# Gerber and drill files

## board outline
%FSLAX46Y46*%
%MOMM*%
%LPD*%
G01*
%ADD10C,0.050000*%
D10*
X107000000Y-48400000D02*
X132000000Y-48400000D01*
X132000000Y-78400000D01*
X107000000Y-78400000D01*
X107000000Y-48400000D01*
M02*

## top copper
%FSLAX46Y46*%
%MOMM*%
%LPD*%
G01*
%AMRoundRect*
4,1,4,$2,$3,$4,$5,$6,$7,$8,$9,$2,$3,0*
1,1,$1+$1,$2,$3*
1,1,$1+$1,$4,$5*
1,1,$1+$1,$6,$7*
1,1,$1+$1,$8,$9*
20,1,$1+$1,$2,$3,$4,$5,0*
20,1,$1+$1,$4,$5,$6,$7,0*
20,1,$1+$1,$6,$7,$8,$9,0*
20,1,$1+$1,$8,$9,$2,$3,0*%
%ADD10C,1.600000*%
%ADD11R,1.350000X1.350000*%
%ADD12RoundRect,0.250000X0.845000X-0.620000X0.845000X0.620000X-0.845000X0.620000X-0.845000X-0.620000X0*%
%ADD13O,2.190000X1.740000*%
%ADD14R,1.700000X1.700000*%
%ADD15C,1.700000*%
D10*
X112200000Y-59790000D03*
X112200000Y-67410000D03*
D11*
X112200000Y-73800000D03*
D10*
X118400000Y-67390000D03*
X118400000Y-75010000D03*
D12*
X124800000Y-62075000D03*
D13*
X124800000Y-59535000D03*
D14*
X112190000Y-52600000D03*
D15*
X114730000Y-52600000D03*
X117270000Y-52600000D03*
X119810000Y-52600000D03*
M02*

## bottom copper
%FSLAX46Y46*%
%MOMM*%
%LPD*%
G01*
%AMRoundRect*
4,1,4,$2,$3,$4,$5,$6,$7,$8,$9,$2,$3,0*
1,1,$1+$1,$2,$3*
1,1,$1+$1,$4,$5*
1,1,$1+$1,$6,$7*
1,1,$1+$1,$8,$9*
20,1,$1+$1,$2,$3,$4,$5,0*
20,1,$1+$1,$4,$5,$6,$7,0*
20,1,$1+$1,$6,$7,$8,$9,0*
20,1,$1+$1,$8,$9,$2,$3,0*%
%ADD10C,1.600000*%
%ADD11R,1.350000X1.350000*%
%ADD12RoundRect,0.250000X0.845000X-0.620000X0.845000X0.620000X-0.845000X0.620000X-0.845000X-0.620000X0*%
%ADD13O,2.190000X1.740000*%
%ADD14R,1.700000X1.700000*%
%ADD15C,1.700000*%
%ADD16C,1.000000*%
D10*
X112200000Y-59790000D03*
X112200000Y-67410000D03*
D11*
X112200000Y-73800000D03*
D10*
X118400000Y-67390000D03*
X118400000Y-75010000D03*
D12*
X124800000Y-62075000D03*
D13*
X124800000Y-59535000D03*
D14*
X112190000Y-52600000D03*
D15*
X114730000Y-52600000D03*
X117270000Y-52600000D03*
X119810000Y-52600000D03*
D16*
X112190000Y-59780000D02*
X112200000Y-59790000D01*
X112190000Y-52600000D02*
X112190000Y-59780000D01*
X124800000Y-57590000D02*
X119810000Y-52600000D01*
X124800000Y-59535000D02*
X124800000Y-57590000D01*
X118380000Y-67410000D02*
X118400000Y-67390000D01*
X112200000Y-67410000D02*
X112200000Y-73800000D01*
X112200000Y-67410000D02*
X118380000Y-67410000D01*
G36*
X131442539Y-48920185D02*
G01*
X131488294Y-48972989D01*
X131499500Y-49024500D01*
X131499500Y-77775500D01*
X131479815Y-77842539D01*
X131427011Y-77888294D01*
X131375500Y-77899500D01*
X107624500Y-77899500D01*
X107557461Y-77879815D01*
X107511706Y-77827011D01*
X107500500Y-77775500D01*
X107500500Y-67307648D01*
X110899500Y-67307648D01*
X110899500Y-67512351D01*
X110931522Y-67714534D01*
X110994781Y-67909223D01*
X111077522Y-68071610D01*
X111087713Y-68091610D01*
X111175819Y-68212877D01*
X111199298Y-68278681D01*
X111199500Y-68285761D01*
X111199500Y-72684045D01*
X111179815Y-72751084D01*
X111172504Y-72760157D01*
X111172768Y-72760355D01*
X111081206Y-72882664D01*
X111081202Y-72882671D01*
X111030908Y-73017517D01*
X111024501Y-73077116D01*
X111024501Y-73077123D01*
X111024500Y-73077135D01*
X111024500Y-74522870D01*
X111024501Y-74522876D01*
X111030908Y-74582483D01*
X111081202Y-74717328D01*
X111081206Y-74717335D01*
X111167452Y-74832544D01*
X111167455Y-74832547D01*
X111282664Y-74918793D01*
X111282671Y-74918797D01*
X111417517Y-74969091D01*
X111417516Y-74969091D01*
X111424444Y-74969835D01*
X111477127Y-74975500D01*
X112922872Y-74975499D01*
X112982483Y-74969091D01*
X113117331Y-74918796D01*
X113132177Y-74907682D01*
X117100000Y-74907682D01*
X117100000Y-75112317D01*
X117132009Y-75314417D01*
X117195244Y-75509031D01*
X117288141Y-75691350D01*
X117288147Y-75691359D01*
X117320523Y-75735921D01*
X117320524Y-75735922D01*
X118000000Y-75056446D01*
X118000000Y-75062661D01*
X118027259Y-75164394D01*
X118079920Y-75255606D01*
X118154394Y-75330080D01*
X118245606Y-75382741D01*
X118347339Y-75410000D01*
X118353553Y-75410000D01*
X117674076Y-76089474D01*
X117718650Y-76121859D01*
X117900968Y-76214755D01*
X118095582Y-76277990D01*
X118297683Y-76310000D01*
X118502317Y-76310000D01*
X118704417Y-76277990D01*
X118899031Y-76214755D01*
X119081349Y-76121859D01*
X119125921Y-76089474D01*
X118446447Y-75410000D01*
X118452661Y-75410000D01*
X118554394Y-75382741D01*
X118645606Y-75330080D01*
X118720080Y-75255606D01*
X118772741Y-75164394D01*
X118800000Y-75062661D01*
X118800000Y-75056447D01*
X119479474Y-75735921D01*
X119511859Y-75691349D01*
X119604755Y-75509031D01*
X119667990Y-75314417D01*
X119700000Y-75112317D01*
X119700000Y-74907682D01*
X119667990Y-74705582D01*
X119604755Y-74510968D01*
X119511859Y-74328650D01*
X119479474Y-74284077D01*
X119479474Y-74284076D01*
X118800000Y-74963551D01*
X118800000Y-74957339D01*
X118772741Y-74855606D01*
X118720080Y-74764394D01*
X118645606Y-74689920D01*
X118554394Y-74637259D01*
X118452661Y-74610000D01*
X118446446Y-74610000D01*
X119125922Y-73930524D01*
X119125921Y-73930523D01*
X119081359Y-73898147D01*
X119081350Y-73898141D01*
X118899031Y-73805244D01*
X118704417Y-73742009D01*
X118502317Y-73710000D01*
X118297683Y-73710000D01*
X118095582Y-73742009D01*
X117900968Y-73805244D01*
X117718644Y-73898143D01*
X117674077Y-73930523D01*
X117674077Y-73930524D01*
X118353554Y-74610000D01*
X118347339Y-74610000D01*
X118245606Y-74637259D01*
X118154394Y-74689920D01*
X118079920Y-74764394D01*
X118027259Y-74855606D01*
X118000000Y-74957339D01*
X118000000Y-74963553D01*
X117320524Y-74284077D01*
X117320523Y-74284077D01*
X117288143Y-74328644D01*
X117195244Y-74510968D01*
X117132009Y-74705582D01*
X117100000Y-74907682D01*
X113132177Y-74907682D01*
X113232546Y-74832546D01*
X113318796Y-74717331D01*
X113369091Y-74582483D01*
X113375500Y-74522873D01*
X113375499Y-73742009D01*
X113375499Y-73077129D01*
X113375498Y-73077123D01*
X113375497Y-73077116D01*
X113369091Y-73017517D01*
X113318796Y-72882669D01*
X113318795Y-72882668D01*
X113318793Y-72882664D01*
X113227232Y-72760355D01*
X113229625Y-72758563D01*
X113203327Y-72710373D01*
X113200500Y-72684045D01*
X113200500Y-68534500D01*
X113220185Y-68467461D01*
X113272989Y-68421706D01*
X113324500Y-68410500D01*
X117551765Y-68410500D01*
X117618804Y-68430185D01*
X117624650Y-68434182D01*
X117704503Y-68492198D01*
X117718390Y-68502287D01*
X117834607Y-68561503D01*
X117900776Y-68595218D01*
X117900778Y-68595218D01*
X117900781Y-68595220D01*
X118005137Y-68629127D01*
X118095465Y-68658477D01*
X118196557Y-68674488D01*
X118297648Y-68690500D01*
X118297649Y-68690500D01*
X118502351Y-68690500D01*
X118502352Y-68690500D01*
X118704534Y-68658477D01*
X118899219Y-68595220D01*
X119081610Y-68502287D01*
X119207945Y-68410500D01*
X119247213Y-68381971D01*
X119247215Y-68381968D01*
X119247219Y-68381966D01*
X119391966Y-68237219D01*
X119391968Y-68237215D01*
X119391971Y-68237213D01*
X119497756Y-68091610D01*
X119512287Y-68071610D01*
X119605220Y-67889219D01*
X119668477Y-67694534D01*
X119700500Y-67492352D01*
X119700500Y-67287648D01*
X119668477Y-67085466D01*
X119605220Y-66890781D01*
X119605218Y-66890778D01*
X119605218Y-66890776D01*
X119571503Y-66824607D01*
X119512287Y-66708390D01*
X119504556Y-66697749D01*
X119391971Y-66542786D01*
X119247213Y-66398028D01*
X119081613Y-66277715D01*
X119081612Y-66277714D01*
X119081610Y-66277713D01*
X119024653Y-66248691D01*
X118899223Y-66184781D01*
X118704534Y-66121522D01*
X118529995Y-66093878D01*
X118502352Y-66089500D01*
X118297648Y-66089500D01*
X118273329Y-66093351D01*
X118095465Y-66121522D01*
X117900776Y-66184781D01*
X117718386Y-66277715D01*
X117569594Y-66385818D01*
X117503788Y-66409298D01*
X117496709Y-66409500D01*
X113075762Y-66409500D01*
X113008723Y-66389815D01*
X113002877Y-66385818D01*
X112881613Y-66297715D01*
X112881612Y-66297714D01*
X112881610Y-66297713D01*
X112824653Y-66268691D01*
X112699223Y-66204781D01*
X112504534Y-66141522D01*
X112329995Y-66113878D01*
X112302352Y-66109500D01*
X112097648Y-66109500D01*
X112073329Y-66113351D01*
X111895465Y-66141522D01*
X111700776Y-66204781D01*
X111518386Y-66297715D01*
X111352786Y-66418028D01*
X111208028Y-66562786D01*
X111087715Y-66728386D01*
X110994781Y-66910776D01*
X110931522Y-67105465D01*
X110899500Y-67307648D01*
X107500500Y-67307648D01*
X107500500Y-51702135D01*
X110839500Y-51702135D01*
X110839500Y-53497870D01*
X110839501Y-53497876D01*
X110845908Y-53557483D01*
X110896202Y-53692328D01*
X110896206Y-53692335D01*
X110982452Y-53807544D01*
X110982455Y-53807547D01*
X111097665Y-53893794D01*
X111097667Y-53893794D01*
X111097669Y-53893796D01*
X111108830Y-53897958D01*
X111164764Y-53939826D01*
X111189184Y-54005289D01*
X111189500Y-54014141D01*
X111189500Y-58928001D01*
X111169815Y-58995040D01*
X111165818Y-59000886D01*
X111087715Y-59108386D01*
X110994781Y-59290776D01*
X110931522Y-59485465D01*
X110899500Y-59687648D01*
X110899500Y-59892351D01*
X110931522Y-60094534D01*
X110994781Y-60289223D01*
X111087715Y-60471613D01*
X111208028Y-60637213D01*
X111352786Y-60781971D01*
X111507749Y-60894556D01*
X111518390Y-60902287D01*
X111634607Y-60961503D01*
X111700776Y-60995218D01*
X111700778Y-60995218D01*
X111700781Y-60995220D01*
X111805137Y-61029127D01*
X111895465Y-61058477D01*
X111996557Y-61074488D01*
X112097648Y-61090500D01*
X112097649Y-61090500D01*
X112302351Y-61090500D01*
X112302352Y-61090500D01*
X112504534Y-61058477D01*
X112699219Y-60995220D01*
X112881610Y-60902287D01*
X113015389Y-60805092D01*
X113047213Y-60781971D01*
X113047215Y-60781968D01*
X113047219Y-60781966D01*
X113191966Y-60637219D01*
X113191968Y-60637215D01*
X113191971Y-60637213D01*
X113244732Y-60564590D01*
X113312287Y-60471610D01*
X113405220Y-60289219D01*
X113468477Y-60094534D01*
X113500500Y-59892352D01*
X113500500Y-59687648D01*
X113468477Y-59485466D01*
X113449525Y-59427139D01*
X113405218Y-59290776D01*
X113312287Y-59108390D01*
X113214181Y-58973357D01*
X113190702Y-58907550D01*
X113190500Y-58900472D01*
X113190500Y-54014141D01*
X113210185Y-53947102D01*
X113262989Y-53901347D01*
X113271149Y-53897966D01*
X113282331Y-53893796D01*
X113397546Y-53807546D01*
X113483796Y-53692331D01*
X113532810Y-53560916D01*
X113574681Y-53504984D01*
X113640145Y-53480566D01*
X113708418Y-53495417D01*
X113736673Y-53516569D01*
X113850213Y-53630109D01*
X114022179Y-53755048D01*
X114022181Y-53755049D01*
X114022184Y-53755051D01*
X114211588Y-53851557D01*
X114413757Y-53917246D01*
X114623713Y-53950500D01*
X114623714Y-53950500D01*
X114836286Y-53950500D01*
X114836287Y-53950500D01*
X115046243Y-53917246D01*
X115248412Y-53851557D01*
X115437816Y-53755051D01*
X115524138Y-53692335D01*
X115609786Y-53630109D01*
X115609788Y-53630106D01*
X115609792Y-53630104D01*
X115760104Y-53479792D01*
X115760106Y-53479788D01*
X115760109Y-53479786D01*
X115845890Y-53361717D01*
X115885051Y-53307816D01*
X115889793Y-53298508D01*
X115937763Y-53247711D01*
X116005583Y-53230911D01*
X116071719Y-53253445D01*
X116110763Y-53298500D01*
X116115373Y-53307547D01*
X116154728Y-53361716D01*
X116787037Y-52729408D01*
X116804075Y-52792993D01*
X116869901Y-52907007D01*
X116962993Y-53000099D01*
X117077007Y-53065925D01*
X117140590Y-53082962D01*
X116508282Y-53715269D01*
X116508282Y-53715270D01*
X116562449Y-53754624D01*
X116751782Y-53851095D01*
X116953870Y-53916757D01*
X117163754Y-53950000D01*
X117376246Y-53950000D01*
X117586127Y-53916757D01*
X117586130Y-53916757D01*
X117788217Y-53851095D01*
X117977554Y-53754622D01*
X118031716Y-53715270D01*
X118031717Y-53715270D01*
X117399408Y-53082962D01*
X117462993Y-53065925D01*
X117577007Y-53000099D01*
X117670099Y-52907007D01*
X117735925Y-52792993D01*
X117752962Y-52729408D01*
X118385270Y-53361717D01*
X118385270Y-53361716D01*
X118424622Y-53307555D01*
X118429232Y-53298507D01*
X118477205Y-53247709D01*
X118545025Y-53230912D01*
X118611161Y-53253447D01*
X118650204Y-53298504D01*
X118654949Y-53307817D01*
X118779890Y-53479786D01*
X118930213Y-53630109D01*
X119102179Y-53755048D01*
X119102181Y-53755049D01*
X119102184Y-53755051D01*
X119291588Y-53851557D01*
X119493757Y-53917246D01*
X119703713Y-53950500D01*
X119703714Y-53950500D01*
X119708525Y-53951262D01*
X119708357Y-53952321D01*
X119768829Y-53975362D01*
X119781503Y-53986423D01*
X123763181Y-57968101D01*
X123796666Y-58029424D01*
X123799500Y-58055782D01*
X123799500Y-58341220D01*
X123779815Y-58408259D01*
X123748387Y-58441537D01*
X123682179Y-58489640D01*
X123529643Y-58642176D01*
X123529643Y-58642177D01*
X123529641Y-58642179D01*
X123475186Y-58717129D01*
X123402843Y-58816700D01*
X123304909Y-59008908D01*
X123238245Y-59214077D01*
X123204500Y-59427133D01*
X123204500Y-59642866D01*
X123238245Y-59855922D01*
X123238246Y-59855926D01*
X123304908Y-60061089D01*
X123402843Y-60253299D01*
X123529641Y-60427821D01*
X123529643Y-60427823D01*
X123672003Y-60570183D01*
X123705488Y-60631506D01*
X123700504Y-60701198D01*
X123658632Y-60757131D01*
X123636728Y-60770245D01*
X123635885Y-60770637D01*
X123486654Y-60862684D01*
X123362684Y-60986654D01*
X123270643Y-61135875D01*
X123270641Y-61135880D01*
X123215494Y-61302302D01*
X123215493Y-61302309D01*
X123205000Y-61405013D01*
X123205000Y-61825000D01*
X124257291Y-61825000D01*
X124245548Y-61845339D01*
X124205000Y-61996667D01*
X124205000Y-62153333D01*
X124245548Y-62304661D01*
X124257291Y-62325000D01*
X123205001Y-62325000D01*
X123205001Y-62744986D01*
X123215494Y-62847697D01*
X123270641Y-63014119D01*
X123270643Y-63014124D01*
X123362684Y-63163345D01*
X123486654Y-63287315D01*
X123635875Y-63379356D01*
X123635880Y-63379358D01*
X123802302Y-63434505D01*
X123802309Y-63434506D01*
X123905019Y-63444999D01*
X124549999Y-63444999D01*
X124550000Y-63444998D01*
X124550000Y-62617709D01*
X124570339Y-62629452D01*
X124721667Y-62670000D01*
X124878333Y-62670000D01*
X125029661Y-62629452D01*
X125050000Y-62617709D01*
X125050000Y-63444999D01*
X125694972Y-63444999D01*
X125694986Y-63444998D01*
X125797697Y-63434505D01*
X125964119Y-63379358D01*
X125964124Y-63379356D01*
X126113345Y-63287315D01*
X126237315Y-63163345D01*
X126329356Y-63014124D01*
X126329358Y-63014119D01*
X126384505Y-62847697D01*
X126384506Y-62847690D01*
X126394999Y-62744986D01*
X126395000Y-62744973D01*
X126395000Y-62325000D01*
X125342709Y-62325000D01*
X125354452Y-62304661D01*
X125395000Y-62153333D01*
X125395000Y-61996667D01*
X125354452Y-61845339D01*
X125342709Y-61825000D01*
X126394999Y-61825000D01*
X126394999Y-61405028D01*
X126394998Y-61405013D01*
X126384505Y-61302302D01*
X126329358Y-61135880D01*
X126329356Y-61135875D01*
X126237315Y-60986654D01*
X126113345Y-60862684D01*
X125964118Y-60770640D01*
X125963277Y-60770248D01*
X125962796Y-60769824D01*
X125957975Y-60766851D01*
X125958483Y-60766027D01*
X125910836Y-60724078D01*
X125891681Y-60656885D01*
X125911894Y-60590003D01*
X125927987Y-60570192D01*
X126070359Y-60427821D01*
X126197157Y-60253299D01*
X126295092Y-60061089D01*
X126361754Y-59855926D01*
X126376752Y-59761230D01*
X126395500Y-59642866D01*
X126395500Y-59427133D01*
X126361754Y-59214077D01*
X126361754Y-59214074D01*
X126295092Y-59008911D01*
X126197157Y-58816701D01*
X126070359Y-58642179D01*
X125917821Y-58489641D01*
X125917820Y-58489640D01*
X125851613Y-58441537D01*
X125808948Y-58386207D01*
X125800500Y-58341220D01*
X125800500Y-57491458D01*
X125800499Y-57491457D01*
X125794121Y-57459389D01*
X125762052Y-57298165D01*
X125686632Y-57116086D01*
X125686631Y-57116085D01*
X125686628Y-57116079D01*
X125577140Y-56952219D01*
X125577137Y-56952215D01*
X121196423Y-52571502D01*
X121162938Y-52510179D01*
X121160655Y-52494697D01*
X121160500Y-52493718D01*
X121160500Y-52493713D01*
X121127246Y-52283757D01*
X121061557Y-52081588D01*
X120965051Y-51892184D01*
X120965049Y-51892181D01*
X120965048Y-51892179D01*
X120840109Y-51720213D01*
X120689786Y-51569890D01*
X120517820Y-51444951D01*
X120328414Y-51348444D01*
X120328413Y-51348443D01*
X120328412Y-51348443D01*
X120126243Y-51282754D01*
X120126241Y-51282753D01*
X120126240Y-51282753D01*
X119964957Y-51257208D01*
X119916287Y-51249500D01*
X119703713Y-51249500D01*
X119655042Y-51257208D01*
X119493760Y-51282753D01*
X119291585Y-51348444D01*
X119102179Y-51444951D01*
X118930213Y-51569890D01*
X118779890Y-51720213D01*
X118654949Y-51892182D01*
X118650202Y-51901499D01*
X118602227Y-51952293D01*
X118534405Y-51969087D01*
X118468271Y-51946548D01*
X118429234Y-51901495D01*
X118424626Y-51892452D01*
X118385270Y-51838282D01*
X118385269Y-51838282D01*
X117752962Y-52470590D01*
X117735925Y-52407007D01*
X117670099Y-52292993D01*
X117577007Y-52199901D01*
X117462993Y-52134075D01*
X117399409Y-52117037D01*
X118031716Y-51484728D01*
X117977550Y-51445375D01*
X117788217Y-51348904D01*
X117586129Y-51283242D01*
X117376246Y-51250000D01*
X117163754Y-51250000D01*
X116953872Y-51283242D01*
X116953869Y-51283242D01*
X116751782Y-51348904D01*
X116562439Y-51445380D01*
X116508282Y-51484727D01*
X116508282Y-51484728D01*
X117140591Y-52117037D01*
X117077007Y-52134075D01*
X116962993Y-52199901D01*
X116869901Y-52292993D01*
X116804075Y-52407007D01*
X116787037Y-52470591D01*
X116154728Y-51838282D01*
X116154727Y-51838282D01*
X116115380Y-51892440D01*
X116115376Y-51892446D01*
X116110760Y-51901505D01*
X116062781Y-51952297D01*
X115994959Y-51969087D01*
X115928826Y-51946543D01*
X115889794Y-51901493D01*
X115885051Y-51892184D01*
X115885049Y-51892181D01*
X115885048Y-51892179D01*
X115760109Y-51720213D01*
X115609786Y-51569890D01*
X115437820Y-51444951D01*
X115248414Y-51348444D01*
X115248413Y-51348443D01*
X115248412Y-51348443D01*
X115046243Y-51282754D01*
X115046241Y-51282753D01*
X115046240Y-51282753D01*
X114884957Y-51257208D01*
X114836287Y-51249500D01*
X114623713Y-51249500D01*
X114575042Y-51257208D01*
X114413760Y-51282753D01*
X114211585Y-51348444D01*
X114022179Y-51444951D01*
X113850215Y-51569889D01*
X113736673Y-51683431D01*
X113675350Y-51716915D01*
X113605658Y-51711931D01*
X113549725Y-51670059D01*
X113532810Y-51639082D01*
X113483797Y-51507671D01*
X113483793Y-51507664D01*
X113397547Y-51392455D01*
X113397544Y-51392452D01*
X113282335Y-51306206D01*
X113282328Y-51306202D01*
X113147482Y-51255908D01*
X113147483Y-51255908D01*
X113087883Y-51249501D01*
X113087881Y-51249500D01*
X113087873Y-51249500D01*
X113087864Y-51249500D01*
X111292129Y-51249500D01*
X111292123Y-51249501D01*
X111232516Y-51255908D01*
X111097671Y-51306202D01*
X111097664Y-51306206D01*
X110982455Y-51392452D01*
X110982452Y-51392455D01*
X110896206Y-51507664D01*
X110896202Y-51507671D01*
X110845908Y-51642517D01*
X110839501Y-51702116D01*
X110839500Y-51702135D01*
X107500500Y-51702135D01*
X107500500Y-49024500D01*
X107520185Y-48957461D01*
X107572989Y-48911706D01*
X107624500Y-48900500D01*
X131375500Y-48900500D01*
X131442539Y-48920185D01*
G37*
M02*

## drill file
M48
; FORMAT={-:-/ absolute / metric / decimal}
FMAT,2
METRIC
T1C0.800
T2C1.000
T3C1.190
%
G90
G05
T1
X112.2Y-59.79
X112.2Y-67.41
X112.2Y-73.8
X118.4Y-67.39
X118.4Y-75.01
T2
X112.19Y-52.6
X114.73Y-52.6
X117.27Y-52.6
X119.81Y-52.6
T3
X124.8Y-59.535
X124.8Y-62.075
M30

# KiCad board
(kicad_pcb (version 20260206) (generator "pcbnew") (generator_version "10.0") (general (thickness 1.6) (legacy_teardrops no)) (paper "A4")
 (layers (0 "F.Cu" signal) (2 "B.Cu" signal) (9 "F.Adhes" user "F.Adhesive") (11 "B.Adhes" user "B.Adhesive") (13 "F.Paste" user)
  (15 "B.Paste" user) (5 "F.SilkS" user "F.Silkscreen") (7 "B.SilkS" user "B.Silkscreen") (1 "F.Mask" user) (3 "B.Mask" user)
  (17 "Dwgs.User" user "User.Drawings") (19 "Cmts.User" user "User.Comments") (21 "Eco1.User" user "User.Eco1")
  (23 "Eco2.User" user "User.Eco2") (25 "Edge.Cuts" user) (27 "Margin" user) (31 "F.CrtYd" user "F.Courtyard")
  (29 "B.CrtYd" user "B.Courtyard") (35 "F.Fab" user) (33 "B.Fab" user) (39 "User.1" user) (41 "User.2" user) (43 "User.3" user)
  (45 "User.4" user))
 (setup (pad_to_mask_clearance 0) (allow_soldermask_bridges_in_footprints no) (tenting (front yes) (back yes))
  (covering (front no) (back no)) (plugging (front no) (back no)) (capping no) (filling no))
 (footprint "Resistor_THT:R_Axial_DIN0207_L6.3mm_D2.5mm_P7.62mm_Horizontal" (layer "F.Cu") (at 112.2 59.79 -90)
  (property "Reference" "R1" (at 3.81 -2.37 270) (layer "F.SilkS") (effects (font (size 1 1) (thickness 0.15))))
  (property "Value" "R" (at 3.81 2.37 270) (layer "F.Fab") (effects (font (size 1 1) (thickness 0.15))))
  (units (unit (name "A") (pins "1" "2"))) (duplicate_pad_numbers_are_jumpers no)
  (pad "1" thru_hole circle (at 0 0 270) (size 1.6 1.6) (drill 0.8) (layers "*.Cu" "*.Mask") (remove_unused_layers no)
   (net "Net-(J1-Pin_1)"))
  (pad "2" thru_hole circle (at 7.62 0 270) (size 1.6 1.6) (drill 0.8) (layers "*.Cu" "*.Mask") (remove_unused_layers no)
   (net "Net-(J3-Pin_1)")))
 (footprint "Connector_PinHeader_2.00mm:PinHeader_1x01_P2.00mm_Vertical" (layer "F.Cu") (at 112.2 73.8 -90)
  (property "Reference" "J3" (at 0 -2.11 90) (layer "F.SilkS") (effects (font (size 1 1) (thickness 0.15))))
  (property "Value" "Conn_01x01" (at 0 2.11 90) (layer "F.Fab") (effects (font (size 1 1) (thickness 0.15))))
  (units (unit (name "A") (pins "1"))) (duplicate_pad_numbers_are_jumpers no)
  (pad "1" thru_hole rect (at 0 0 270) (size 1.35 1.35) (drill 0.8) (layers "*.Cu" "*.Mask") (remove_unused_layers no)
   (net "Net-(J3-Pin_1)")))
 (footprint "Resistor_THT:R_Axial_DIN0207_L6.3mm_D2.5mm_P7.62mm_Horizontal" (layer "F.Cu") (at 118.4 67.39 -90)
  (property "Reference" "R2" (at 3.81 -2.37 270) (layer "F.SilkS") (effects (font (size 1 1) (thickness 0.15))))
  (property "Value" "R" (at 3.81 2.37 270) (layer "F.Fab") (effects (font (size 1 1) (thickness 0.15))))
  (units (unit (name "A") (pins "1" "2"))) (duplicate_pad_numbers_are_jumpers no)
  (pad "1" thru_hole circle (at 0 0 270) (size 1.6 1.6) (drill 0.8) (layers "*.Cu" "*.Mask") (remove_unused_layers no)
   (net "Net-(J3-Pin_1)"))
  (pad "2" thru_hole circle (at 7.62 0 270) (size 1.6 1.6) (drill 0.8) (layers "*.Cu" "*.Mask") (remove_unused_layers no) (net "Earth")))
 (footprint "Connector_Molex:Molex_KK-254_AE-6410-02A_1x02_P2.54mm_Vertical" (layer "F.Cu") (at 124.8 62.075 90)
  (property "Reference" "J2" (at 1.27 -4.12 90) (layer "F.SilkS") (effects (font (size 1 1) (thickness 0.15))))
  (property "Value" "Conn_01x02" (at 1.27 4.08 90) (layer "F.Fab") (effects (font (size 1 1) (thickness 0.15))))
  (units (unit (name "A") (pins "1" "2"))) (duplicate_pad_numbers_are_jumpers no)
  (pad "1" thru_hole roundrect (at 0 0 90) (size 1.74 2.19) (drill 1.19) (layers "*.Cu" "*.Mask") (remove_unused_layers no)
   (roundrect_rratio 0.143678) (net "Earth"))
  (pad "2" thru_hole oval (at 2.54 0 90) (size 1.74 2.19) (drill 1.19) (layers "*.Cu" "*.Mask") (remove_unused_layers no)
   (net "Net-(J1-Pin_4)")))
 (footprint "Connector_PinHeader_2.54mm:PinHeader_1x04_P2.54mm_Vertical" (layer "F.Cu") (at 112.19 52.6 90)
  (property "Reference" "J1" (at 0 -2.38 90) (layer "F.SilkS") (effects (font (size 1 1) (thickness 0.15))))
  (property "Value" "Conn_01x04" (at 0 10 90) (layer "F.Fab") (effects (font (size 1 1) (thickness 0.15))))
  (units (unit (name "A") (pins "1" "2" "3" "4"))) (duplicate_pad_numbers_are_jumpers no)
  (pad "1" thru_hole rect (at 0 0 90) (size 1.7 1.7) (drill 1) (layers "*.Cu" "*.Mask") (remove_unused_layers no) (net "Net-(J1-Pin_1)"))
  (pad "2" thru_hole circle (at 0 2.54 90) (size 1.7 1.7) (drill 1) (layers "*.Cu" "*.Mask") (remove_unused_layers no)
   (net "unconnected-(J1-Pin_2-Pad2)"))
  (pad "3" thru_hole circle (at 0 5.08 90) (size 1.7 1.7) (drill 1) (layers "*.Cu" "*.Mask") (remove_unused_layers no) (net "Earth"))
  (pad "4" thru_hole circle (at 0 7.62 90) (size 1.7 1.7) (drill 1) (layers "*.Cu" "*.Mask") (remove_unused_layers no)
   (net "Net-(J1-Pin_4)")))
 (gr_rect (start 107 48.4) (end 132 78.4) (stroke (width 0.05) (type solid)) (fill no) (layer "Edge.Cuts"))
 (segment (start 112.19 59.78) (end 112.2 59.79) (width 1) (layer "B.Cu") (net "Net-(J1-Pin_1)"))
 (segment (start 112.19 52.6) (end 112.19 59.78) (width 1) (layer "B.Cu") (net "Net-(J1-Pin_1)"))
 (segment (start 124.8 57.59) (end 119.81 52.6) (width 1) (layer "B.Cu") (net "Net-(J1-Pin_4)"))
 (segment (start 124.8 59.535) (end 124.8 57.59) (width 1) (layer "B.Cu") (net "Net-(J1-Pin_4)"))
 (segment (start 118.38 67.41) (end 118.4 67.39) (width 1) (layer "B.Cu") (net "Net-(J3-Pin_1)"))
 (segment (start 112.2 67.41) (end 112.2 73.8) (width 1) (layer "B.Cu") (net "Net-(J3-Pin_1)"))
 (segment (start 112.2 67.41) (end 118.38 67.41) (width 1) (layer "B.Cu") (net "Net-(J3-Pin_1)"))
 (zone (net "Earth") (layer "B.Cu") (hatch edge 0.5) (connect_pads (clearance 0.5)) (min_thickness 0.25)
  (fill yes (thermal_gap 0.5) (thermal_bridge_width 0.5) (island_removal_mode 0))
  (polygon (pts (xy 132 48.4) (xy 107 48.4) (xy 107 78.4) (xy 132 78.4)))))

